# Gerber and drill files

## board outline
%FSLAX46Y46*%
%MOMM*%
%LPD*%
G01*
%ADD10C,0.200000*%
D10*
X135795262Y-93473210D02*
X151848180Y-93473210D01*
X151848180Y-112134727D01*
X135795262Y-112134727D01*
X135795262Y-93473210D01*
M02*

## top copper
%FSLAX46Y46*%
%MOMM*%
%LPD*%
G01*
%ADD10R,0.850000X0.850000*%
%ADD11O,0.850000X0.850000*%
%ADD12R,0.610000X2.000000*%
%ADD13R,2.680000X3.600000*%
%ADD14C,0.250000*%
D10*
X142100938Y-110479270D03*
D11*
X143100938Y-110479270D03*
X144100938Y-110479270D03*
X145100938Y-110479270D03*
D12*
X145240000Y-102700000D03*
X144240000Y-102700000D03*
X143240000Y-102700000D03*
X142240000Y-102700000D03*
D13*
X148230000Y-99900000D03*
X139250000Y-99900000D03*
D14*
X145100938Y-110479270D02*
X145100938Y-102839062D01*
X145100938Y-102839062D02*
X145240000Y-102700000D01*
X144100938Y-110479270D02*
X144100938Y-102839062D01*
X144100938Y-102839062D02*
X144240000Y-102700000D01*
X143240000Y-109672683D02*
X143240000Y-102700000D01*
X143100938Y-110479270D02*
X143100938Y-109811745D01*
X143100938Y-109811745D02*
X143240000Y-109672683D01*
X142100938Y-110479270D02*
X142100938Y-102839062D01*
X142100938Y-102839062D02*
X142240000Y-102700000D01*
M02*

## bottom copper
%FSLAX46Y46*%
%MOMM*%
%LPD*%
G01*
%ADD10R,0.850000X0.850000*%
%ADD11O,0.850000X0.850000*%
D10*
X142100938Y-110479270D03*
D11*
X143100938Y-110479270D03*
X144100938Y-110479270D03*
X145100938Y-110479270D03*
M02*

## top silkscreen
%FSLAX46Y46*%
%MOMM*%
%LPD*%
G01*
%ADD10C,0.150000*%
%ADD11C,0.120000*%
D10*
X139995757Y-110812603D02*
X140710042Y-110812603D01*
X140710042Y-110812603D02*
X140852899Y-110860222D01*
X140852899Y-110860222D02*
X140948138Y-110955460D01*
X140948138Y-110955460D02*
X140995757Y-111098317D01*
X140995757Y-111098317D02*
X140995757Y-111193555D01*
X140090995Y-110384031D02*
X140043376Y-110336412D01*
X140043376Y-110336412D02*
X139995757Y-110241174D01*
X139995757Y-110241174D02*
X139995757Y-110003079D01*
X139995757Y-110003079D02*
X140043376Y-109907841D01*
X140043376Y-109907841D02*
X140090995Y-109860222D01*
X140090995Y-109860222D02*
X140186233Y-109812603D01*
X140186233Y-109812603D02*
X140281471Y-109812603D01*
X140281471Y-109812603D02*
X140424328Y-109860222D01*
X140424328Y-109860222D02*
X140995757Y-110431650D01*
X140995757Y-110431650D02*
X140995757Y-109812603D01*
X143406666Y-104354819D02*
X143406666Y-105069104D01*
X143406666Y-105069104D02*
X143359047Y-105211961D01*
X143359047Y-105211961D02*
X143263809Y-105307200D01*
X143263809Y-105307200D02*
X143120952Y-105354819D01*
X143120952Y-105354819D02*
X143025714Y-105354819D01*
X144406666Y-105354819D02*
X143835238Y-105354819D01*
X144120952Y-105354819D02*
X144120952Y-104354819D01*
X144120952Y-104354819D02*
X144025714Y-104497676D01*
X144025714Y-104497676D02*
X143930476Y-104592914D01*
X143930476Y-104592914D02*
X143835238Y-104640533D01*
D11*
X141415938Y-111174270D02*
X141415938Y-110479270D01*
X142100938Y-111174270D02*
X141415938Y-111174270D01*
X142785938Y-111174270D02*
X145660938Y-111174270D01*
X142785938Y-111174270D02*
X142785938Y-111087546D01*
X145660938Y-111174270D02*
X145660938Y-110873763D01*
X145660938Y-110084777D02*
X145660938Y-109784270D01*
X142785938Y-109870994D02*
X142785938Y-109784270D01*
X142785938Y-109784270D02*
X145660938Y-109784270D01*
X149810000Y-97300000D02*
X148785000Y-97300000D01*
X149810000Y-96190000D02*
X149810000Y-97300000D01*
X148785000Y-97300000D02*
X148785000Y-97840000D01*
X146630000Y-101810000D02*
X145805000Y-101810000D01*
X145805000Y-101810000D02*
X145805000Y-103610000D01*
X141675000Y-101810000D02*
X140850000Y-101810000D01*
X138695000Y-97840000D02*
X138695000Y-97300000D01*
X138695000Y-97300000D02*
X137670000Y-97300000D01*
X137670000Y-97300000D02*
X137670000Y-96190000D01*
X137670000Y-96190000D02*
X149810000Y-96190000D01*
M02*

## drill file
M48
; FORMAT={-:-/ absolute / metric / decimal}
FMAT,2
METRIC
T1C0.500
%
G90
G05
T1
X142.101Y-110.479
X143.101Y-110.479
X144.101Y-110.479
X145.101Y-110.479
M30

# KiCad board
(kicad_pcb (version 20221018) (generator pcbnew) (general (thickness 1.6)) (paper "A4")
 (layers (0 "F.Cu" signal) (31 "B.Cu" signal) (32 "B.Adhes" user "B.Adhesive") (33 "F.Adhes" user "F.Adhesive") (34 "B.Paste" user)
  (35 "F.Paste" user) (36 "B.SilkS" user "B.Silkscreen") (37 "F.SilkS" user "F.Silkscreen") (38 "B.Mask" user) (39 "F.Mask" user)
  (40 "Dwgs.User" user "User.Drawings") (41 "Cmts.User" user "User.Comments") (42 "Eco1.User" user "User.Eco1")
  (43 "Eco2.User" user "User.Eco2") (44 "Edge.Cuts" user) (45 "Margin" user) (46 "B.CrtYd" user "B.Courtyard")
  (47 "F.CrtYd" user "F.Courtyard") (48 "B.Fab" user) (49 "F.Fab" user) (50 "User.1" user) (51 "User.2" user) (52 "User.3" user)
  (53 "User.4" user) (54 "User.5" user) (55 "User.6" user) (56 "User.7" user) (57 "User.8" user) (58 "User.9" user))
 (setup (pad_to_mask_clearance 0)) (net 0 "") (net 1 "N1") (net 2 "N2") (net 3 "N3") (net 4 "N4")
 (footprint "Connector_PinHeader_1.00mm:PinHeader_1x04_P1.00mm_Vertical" (layer "F.Cu") (at 142.100938 110.47927 90)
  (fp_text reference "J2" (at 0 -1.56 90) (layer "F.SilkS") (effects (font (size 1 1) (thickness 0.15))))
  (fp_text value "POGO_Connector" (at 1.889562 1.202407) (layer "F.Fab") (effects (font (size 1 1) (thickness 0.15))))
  (fp_line (start -0.695 -0.685) (end 0 -0.685) (stroke (width 0.12) (type solid)) (layer "F.SilkS"))
  (fp_line (start -0.695 0) (end -0.695 -0.685) (stroke (width 0.12) (type solid)) (layer "F.SilkS"))
  (fp_line (start -0.695 0.685) (end -0.695 3.56) (stroke (width 0.12) (type solid)) (layer "F.SilkS"))
  (fp_line (start -0.695 0.685) (end -0.608276 0.685) (stroke (width 0.12) (type solid)) (layer "F.SilkS"))
  (fp_line (start -0.695 3.56) (end -0.394493 3.56) (stroke (width 0.12) (type solid)) (layer "F.SilkS"))
  (fp_line (start 0.394493 3.56) (end 0.695 3.56) (stroke (width 0.12) (type solid)) (layer "F.SilkS"))
  (fp_line (start 0.608276 0.685) (end 0.695 0.685) (stroke (width 0.12) (type solid)) (layer "F.SilkS"))
  (fp_line (start 0.695 0.685) (end 0.695 3.56) (stroke (width 0.12) (type solid)) (layer "F.SilkS"))
  (pad "1" thru_hole rect (at 0 0 90) (size 0.85 0.85) (drill 0.5) (layers "*.Cu" "*.Mask") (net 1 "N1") (clearance 0.15))
  (pad "2" thru_hole oval (at 0 1 90) (size 0.85 0.85) (drill 0.5) (layers "*.Cu" "*.Mask") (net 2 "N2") (clearance 0.15))
  (pad "3" thru_hole oval (at 0 2 90) (size 0.85 0.85) (drill 0.5) (layers "*.Cu" "*.Mask") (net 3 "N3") (clearance 0.15))
  (pad "4" thru_hole oval (at 0 3 90) (size 0.85 0.85) (drill 0.5) (layers "*.Cu" "*.Mask") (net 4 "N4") (clearance 0.15)))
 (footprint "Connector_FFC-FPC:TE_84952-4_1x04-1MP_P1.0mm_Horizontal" (layer "F.Cu") (at 143.74 100.9 180)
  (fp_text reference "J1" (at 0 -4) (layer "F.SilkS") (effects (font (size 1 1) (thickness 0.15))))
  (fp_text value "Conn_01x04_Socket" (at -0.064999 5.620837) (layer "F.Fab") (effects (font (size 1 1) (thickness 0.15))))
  (fp_line (start -6.07 3.6) (end -5.045 3.6) (stroke (width 0.12) (type solid)) (layer "F.SilkS"))
  (fp_line (start -6.07 4.71) (end -6.07 3.6) (stroke (width 0.12) (type solid)) (layer "F.SilkS"))
  (fp_line (start -5.045 3.6) (end -5.045 3.06) (stroke (width 0.12) (type solid)) (layer "F.SilkS"))
  (fp_line (start -2.89 -0.91) (end -2.065 -0.91) (stroke (width 0.12) (type solid)) (layer "F.SilkS"))
  (fp_line (start -2.065 -0.91) (end -2.065 -2.71) (stroke (width 0.12) (type solid)) (layer "F.SilkS"))
  (fp_line (start 2.065 -0.91) (end 2.89 -0.91) (stroke (width 0.12) (type solid)) (layer "F.SilkS"))
  (fp_line (start 5.045 3.06) (end 5.045 3.6) (stroke (width 0.12) (type solid)) (layer "F.SilkS"))
  (fp_line (start 5.045 3.6) (end 6.07 3.6) (stroke (width 0.12) (type solid)) (layer "F.SilkS"))
  (fp_line (start 6.07 3.6) (end 6.07 4.71) (stroke (width 0.12) (type solid)) (layer "F.SilkS"))
  (fp_line (start 6.07 4.71) (end -6.07 4.71) (stroke (width 0.12) (type solid)) (layer "F.SilkS"))
  (pad "1" smd rect (at -1.5 -1.8 180) (size 0.61 2) (layers "F.Cu" "F.Paste" "F.Mask") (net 4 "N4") (clearance 0.15))
  (pad "2" smd rect (at -0.5 -1.8 180) (size 0.61 2) (layers "F.Cu" "F.Paste" "F.Mask") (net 3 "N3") (clearance 0.15))
  (pad "3" smd rect (at 0.5 -1.8 180) (size 0.61 2) (layers "F.Cu" "F.Paste" "F.Mask") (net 2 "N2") (clearance 0.15))
  (pad "4" smd rect (at 1.5 -1.8 180) (size 0.61 2) (layers "F.Cu" "F.Paste" "F.Mask") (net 1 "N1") (clearance 0.15))
  (pad "MP" smd rect (at -4.49 1 180) (size 2.68 3.6) (layers "F.Cu" "F.Paste" "F.Mask"))
  (pad "MP" smd rect (at 4.49 1 180) (size 2.68 3.6) (layers "F.Cu" "F.Paste" "F.Mask")))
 (gr_rect (start 135.795262 93.47321) (end 151.84818 112.134727) (stroke (width 0.2) (type default)) (fill none) (layer "Edge.Cuts"))
 (segment (start 145.100938 110.47927) (end 145.100938 102.839062) (width 0.25) (layer "F.Cu") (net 4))
 (segment (start 145.100938 102.839062) (end 145.24 102.7) (width 0.25) (layer "F.Cu") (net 4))
 (segment (start 144.100938 110.47927) (end 144.100938 102.839062) (width 0.25) (layer "F.Cu") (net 3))
 (segment (start 144.100938 102.839062) (end 144.24 102.7) (width 0.25) (layer "F.Cu") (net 3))
 (segment (start 143.24 109.672683) (end 143.24 102.7) (width 0.25) (layer "F.Cu") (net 2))
 (segment (start 143.100938 110.47927) (end 143.100938 109.811745) (width 0.25) (layer "F.Cu") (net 2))
 (segment (start 143.100938 109.811745) (end 143.24 109.672683) (width 0.25) (layer "F.Cu") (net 2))
 (segment (start 142.100938 110.47927) (end 142.100938 102.839062) (width 0.25) (layer "F.Cu") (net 1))
 (segment (start 142.100938 102.839062) (end 142.24 102.7) (width 0.25) (layer "F.Cu") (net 1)))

